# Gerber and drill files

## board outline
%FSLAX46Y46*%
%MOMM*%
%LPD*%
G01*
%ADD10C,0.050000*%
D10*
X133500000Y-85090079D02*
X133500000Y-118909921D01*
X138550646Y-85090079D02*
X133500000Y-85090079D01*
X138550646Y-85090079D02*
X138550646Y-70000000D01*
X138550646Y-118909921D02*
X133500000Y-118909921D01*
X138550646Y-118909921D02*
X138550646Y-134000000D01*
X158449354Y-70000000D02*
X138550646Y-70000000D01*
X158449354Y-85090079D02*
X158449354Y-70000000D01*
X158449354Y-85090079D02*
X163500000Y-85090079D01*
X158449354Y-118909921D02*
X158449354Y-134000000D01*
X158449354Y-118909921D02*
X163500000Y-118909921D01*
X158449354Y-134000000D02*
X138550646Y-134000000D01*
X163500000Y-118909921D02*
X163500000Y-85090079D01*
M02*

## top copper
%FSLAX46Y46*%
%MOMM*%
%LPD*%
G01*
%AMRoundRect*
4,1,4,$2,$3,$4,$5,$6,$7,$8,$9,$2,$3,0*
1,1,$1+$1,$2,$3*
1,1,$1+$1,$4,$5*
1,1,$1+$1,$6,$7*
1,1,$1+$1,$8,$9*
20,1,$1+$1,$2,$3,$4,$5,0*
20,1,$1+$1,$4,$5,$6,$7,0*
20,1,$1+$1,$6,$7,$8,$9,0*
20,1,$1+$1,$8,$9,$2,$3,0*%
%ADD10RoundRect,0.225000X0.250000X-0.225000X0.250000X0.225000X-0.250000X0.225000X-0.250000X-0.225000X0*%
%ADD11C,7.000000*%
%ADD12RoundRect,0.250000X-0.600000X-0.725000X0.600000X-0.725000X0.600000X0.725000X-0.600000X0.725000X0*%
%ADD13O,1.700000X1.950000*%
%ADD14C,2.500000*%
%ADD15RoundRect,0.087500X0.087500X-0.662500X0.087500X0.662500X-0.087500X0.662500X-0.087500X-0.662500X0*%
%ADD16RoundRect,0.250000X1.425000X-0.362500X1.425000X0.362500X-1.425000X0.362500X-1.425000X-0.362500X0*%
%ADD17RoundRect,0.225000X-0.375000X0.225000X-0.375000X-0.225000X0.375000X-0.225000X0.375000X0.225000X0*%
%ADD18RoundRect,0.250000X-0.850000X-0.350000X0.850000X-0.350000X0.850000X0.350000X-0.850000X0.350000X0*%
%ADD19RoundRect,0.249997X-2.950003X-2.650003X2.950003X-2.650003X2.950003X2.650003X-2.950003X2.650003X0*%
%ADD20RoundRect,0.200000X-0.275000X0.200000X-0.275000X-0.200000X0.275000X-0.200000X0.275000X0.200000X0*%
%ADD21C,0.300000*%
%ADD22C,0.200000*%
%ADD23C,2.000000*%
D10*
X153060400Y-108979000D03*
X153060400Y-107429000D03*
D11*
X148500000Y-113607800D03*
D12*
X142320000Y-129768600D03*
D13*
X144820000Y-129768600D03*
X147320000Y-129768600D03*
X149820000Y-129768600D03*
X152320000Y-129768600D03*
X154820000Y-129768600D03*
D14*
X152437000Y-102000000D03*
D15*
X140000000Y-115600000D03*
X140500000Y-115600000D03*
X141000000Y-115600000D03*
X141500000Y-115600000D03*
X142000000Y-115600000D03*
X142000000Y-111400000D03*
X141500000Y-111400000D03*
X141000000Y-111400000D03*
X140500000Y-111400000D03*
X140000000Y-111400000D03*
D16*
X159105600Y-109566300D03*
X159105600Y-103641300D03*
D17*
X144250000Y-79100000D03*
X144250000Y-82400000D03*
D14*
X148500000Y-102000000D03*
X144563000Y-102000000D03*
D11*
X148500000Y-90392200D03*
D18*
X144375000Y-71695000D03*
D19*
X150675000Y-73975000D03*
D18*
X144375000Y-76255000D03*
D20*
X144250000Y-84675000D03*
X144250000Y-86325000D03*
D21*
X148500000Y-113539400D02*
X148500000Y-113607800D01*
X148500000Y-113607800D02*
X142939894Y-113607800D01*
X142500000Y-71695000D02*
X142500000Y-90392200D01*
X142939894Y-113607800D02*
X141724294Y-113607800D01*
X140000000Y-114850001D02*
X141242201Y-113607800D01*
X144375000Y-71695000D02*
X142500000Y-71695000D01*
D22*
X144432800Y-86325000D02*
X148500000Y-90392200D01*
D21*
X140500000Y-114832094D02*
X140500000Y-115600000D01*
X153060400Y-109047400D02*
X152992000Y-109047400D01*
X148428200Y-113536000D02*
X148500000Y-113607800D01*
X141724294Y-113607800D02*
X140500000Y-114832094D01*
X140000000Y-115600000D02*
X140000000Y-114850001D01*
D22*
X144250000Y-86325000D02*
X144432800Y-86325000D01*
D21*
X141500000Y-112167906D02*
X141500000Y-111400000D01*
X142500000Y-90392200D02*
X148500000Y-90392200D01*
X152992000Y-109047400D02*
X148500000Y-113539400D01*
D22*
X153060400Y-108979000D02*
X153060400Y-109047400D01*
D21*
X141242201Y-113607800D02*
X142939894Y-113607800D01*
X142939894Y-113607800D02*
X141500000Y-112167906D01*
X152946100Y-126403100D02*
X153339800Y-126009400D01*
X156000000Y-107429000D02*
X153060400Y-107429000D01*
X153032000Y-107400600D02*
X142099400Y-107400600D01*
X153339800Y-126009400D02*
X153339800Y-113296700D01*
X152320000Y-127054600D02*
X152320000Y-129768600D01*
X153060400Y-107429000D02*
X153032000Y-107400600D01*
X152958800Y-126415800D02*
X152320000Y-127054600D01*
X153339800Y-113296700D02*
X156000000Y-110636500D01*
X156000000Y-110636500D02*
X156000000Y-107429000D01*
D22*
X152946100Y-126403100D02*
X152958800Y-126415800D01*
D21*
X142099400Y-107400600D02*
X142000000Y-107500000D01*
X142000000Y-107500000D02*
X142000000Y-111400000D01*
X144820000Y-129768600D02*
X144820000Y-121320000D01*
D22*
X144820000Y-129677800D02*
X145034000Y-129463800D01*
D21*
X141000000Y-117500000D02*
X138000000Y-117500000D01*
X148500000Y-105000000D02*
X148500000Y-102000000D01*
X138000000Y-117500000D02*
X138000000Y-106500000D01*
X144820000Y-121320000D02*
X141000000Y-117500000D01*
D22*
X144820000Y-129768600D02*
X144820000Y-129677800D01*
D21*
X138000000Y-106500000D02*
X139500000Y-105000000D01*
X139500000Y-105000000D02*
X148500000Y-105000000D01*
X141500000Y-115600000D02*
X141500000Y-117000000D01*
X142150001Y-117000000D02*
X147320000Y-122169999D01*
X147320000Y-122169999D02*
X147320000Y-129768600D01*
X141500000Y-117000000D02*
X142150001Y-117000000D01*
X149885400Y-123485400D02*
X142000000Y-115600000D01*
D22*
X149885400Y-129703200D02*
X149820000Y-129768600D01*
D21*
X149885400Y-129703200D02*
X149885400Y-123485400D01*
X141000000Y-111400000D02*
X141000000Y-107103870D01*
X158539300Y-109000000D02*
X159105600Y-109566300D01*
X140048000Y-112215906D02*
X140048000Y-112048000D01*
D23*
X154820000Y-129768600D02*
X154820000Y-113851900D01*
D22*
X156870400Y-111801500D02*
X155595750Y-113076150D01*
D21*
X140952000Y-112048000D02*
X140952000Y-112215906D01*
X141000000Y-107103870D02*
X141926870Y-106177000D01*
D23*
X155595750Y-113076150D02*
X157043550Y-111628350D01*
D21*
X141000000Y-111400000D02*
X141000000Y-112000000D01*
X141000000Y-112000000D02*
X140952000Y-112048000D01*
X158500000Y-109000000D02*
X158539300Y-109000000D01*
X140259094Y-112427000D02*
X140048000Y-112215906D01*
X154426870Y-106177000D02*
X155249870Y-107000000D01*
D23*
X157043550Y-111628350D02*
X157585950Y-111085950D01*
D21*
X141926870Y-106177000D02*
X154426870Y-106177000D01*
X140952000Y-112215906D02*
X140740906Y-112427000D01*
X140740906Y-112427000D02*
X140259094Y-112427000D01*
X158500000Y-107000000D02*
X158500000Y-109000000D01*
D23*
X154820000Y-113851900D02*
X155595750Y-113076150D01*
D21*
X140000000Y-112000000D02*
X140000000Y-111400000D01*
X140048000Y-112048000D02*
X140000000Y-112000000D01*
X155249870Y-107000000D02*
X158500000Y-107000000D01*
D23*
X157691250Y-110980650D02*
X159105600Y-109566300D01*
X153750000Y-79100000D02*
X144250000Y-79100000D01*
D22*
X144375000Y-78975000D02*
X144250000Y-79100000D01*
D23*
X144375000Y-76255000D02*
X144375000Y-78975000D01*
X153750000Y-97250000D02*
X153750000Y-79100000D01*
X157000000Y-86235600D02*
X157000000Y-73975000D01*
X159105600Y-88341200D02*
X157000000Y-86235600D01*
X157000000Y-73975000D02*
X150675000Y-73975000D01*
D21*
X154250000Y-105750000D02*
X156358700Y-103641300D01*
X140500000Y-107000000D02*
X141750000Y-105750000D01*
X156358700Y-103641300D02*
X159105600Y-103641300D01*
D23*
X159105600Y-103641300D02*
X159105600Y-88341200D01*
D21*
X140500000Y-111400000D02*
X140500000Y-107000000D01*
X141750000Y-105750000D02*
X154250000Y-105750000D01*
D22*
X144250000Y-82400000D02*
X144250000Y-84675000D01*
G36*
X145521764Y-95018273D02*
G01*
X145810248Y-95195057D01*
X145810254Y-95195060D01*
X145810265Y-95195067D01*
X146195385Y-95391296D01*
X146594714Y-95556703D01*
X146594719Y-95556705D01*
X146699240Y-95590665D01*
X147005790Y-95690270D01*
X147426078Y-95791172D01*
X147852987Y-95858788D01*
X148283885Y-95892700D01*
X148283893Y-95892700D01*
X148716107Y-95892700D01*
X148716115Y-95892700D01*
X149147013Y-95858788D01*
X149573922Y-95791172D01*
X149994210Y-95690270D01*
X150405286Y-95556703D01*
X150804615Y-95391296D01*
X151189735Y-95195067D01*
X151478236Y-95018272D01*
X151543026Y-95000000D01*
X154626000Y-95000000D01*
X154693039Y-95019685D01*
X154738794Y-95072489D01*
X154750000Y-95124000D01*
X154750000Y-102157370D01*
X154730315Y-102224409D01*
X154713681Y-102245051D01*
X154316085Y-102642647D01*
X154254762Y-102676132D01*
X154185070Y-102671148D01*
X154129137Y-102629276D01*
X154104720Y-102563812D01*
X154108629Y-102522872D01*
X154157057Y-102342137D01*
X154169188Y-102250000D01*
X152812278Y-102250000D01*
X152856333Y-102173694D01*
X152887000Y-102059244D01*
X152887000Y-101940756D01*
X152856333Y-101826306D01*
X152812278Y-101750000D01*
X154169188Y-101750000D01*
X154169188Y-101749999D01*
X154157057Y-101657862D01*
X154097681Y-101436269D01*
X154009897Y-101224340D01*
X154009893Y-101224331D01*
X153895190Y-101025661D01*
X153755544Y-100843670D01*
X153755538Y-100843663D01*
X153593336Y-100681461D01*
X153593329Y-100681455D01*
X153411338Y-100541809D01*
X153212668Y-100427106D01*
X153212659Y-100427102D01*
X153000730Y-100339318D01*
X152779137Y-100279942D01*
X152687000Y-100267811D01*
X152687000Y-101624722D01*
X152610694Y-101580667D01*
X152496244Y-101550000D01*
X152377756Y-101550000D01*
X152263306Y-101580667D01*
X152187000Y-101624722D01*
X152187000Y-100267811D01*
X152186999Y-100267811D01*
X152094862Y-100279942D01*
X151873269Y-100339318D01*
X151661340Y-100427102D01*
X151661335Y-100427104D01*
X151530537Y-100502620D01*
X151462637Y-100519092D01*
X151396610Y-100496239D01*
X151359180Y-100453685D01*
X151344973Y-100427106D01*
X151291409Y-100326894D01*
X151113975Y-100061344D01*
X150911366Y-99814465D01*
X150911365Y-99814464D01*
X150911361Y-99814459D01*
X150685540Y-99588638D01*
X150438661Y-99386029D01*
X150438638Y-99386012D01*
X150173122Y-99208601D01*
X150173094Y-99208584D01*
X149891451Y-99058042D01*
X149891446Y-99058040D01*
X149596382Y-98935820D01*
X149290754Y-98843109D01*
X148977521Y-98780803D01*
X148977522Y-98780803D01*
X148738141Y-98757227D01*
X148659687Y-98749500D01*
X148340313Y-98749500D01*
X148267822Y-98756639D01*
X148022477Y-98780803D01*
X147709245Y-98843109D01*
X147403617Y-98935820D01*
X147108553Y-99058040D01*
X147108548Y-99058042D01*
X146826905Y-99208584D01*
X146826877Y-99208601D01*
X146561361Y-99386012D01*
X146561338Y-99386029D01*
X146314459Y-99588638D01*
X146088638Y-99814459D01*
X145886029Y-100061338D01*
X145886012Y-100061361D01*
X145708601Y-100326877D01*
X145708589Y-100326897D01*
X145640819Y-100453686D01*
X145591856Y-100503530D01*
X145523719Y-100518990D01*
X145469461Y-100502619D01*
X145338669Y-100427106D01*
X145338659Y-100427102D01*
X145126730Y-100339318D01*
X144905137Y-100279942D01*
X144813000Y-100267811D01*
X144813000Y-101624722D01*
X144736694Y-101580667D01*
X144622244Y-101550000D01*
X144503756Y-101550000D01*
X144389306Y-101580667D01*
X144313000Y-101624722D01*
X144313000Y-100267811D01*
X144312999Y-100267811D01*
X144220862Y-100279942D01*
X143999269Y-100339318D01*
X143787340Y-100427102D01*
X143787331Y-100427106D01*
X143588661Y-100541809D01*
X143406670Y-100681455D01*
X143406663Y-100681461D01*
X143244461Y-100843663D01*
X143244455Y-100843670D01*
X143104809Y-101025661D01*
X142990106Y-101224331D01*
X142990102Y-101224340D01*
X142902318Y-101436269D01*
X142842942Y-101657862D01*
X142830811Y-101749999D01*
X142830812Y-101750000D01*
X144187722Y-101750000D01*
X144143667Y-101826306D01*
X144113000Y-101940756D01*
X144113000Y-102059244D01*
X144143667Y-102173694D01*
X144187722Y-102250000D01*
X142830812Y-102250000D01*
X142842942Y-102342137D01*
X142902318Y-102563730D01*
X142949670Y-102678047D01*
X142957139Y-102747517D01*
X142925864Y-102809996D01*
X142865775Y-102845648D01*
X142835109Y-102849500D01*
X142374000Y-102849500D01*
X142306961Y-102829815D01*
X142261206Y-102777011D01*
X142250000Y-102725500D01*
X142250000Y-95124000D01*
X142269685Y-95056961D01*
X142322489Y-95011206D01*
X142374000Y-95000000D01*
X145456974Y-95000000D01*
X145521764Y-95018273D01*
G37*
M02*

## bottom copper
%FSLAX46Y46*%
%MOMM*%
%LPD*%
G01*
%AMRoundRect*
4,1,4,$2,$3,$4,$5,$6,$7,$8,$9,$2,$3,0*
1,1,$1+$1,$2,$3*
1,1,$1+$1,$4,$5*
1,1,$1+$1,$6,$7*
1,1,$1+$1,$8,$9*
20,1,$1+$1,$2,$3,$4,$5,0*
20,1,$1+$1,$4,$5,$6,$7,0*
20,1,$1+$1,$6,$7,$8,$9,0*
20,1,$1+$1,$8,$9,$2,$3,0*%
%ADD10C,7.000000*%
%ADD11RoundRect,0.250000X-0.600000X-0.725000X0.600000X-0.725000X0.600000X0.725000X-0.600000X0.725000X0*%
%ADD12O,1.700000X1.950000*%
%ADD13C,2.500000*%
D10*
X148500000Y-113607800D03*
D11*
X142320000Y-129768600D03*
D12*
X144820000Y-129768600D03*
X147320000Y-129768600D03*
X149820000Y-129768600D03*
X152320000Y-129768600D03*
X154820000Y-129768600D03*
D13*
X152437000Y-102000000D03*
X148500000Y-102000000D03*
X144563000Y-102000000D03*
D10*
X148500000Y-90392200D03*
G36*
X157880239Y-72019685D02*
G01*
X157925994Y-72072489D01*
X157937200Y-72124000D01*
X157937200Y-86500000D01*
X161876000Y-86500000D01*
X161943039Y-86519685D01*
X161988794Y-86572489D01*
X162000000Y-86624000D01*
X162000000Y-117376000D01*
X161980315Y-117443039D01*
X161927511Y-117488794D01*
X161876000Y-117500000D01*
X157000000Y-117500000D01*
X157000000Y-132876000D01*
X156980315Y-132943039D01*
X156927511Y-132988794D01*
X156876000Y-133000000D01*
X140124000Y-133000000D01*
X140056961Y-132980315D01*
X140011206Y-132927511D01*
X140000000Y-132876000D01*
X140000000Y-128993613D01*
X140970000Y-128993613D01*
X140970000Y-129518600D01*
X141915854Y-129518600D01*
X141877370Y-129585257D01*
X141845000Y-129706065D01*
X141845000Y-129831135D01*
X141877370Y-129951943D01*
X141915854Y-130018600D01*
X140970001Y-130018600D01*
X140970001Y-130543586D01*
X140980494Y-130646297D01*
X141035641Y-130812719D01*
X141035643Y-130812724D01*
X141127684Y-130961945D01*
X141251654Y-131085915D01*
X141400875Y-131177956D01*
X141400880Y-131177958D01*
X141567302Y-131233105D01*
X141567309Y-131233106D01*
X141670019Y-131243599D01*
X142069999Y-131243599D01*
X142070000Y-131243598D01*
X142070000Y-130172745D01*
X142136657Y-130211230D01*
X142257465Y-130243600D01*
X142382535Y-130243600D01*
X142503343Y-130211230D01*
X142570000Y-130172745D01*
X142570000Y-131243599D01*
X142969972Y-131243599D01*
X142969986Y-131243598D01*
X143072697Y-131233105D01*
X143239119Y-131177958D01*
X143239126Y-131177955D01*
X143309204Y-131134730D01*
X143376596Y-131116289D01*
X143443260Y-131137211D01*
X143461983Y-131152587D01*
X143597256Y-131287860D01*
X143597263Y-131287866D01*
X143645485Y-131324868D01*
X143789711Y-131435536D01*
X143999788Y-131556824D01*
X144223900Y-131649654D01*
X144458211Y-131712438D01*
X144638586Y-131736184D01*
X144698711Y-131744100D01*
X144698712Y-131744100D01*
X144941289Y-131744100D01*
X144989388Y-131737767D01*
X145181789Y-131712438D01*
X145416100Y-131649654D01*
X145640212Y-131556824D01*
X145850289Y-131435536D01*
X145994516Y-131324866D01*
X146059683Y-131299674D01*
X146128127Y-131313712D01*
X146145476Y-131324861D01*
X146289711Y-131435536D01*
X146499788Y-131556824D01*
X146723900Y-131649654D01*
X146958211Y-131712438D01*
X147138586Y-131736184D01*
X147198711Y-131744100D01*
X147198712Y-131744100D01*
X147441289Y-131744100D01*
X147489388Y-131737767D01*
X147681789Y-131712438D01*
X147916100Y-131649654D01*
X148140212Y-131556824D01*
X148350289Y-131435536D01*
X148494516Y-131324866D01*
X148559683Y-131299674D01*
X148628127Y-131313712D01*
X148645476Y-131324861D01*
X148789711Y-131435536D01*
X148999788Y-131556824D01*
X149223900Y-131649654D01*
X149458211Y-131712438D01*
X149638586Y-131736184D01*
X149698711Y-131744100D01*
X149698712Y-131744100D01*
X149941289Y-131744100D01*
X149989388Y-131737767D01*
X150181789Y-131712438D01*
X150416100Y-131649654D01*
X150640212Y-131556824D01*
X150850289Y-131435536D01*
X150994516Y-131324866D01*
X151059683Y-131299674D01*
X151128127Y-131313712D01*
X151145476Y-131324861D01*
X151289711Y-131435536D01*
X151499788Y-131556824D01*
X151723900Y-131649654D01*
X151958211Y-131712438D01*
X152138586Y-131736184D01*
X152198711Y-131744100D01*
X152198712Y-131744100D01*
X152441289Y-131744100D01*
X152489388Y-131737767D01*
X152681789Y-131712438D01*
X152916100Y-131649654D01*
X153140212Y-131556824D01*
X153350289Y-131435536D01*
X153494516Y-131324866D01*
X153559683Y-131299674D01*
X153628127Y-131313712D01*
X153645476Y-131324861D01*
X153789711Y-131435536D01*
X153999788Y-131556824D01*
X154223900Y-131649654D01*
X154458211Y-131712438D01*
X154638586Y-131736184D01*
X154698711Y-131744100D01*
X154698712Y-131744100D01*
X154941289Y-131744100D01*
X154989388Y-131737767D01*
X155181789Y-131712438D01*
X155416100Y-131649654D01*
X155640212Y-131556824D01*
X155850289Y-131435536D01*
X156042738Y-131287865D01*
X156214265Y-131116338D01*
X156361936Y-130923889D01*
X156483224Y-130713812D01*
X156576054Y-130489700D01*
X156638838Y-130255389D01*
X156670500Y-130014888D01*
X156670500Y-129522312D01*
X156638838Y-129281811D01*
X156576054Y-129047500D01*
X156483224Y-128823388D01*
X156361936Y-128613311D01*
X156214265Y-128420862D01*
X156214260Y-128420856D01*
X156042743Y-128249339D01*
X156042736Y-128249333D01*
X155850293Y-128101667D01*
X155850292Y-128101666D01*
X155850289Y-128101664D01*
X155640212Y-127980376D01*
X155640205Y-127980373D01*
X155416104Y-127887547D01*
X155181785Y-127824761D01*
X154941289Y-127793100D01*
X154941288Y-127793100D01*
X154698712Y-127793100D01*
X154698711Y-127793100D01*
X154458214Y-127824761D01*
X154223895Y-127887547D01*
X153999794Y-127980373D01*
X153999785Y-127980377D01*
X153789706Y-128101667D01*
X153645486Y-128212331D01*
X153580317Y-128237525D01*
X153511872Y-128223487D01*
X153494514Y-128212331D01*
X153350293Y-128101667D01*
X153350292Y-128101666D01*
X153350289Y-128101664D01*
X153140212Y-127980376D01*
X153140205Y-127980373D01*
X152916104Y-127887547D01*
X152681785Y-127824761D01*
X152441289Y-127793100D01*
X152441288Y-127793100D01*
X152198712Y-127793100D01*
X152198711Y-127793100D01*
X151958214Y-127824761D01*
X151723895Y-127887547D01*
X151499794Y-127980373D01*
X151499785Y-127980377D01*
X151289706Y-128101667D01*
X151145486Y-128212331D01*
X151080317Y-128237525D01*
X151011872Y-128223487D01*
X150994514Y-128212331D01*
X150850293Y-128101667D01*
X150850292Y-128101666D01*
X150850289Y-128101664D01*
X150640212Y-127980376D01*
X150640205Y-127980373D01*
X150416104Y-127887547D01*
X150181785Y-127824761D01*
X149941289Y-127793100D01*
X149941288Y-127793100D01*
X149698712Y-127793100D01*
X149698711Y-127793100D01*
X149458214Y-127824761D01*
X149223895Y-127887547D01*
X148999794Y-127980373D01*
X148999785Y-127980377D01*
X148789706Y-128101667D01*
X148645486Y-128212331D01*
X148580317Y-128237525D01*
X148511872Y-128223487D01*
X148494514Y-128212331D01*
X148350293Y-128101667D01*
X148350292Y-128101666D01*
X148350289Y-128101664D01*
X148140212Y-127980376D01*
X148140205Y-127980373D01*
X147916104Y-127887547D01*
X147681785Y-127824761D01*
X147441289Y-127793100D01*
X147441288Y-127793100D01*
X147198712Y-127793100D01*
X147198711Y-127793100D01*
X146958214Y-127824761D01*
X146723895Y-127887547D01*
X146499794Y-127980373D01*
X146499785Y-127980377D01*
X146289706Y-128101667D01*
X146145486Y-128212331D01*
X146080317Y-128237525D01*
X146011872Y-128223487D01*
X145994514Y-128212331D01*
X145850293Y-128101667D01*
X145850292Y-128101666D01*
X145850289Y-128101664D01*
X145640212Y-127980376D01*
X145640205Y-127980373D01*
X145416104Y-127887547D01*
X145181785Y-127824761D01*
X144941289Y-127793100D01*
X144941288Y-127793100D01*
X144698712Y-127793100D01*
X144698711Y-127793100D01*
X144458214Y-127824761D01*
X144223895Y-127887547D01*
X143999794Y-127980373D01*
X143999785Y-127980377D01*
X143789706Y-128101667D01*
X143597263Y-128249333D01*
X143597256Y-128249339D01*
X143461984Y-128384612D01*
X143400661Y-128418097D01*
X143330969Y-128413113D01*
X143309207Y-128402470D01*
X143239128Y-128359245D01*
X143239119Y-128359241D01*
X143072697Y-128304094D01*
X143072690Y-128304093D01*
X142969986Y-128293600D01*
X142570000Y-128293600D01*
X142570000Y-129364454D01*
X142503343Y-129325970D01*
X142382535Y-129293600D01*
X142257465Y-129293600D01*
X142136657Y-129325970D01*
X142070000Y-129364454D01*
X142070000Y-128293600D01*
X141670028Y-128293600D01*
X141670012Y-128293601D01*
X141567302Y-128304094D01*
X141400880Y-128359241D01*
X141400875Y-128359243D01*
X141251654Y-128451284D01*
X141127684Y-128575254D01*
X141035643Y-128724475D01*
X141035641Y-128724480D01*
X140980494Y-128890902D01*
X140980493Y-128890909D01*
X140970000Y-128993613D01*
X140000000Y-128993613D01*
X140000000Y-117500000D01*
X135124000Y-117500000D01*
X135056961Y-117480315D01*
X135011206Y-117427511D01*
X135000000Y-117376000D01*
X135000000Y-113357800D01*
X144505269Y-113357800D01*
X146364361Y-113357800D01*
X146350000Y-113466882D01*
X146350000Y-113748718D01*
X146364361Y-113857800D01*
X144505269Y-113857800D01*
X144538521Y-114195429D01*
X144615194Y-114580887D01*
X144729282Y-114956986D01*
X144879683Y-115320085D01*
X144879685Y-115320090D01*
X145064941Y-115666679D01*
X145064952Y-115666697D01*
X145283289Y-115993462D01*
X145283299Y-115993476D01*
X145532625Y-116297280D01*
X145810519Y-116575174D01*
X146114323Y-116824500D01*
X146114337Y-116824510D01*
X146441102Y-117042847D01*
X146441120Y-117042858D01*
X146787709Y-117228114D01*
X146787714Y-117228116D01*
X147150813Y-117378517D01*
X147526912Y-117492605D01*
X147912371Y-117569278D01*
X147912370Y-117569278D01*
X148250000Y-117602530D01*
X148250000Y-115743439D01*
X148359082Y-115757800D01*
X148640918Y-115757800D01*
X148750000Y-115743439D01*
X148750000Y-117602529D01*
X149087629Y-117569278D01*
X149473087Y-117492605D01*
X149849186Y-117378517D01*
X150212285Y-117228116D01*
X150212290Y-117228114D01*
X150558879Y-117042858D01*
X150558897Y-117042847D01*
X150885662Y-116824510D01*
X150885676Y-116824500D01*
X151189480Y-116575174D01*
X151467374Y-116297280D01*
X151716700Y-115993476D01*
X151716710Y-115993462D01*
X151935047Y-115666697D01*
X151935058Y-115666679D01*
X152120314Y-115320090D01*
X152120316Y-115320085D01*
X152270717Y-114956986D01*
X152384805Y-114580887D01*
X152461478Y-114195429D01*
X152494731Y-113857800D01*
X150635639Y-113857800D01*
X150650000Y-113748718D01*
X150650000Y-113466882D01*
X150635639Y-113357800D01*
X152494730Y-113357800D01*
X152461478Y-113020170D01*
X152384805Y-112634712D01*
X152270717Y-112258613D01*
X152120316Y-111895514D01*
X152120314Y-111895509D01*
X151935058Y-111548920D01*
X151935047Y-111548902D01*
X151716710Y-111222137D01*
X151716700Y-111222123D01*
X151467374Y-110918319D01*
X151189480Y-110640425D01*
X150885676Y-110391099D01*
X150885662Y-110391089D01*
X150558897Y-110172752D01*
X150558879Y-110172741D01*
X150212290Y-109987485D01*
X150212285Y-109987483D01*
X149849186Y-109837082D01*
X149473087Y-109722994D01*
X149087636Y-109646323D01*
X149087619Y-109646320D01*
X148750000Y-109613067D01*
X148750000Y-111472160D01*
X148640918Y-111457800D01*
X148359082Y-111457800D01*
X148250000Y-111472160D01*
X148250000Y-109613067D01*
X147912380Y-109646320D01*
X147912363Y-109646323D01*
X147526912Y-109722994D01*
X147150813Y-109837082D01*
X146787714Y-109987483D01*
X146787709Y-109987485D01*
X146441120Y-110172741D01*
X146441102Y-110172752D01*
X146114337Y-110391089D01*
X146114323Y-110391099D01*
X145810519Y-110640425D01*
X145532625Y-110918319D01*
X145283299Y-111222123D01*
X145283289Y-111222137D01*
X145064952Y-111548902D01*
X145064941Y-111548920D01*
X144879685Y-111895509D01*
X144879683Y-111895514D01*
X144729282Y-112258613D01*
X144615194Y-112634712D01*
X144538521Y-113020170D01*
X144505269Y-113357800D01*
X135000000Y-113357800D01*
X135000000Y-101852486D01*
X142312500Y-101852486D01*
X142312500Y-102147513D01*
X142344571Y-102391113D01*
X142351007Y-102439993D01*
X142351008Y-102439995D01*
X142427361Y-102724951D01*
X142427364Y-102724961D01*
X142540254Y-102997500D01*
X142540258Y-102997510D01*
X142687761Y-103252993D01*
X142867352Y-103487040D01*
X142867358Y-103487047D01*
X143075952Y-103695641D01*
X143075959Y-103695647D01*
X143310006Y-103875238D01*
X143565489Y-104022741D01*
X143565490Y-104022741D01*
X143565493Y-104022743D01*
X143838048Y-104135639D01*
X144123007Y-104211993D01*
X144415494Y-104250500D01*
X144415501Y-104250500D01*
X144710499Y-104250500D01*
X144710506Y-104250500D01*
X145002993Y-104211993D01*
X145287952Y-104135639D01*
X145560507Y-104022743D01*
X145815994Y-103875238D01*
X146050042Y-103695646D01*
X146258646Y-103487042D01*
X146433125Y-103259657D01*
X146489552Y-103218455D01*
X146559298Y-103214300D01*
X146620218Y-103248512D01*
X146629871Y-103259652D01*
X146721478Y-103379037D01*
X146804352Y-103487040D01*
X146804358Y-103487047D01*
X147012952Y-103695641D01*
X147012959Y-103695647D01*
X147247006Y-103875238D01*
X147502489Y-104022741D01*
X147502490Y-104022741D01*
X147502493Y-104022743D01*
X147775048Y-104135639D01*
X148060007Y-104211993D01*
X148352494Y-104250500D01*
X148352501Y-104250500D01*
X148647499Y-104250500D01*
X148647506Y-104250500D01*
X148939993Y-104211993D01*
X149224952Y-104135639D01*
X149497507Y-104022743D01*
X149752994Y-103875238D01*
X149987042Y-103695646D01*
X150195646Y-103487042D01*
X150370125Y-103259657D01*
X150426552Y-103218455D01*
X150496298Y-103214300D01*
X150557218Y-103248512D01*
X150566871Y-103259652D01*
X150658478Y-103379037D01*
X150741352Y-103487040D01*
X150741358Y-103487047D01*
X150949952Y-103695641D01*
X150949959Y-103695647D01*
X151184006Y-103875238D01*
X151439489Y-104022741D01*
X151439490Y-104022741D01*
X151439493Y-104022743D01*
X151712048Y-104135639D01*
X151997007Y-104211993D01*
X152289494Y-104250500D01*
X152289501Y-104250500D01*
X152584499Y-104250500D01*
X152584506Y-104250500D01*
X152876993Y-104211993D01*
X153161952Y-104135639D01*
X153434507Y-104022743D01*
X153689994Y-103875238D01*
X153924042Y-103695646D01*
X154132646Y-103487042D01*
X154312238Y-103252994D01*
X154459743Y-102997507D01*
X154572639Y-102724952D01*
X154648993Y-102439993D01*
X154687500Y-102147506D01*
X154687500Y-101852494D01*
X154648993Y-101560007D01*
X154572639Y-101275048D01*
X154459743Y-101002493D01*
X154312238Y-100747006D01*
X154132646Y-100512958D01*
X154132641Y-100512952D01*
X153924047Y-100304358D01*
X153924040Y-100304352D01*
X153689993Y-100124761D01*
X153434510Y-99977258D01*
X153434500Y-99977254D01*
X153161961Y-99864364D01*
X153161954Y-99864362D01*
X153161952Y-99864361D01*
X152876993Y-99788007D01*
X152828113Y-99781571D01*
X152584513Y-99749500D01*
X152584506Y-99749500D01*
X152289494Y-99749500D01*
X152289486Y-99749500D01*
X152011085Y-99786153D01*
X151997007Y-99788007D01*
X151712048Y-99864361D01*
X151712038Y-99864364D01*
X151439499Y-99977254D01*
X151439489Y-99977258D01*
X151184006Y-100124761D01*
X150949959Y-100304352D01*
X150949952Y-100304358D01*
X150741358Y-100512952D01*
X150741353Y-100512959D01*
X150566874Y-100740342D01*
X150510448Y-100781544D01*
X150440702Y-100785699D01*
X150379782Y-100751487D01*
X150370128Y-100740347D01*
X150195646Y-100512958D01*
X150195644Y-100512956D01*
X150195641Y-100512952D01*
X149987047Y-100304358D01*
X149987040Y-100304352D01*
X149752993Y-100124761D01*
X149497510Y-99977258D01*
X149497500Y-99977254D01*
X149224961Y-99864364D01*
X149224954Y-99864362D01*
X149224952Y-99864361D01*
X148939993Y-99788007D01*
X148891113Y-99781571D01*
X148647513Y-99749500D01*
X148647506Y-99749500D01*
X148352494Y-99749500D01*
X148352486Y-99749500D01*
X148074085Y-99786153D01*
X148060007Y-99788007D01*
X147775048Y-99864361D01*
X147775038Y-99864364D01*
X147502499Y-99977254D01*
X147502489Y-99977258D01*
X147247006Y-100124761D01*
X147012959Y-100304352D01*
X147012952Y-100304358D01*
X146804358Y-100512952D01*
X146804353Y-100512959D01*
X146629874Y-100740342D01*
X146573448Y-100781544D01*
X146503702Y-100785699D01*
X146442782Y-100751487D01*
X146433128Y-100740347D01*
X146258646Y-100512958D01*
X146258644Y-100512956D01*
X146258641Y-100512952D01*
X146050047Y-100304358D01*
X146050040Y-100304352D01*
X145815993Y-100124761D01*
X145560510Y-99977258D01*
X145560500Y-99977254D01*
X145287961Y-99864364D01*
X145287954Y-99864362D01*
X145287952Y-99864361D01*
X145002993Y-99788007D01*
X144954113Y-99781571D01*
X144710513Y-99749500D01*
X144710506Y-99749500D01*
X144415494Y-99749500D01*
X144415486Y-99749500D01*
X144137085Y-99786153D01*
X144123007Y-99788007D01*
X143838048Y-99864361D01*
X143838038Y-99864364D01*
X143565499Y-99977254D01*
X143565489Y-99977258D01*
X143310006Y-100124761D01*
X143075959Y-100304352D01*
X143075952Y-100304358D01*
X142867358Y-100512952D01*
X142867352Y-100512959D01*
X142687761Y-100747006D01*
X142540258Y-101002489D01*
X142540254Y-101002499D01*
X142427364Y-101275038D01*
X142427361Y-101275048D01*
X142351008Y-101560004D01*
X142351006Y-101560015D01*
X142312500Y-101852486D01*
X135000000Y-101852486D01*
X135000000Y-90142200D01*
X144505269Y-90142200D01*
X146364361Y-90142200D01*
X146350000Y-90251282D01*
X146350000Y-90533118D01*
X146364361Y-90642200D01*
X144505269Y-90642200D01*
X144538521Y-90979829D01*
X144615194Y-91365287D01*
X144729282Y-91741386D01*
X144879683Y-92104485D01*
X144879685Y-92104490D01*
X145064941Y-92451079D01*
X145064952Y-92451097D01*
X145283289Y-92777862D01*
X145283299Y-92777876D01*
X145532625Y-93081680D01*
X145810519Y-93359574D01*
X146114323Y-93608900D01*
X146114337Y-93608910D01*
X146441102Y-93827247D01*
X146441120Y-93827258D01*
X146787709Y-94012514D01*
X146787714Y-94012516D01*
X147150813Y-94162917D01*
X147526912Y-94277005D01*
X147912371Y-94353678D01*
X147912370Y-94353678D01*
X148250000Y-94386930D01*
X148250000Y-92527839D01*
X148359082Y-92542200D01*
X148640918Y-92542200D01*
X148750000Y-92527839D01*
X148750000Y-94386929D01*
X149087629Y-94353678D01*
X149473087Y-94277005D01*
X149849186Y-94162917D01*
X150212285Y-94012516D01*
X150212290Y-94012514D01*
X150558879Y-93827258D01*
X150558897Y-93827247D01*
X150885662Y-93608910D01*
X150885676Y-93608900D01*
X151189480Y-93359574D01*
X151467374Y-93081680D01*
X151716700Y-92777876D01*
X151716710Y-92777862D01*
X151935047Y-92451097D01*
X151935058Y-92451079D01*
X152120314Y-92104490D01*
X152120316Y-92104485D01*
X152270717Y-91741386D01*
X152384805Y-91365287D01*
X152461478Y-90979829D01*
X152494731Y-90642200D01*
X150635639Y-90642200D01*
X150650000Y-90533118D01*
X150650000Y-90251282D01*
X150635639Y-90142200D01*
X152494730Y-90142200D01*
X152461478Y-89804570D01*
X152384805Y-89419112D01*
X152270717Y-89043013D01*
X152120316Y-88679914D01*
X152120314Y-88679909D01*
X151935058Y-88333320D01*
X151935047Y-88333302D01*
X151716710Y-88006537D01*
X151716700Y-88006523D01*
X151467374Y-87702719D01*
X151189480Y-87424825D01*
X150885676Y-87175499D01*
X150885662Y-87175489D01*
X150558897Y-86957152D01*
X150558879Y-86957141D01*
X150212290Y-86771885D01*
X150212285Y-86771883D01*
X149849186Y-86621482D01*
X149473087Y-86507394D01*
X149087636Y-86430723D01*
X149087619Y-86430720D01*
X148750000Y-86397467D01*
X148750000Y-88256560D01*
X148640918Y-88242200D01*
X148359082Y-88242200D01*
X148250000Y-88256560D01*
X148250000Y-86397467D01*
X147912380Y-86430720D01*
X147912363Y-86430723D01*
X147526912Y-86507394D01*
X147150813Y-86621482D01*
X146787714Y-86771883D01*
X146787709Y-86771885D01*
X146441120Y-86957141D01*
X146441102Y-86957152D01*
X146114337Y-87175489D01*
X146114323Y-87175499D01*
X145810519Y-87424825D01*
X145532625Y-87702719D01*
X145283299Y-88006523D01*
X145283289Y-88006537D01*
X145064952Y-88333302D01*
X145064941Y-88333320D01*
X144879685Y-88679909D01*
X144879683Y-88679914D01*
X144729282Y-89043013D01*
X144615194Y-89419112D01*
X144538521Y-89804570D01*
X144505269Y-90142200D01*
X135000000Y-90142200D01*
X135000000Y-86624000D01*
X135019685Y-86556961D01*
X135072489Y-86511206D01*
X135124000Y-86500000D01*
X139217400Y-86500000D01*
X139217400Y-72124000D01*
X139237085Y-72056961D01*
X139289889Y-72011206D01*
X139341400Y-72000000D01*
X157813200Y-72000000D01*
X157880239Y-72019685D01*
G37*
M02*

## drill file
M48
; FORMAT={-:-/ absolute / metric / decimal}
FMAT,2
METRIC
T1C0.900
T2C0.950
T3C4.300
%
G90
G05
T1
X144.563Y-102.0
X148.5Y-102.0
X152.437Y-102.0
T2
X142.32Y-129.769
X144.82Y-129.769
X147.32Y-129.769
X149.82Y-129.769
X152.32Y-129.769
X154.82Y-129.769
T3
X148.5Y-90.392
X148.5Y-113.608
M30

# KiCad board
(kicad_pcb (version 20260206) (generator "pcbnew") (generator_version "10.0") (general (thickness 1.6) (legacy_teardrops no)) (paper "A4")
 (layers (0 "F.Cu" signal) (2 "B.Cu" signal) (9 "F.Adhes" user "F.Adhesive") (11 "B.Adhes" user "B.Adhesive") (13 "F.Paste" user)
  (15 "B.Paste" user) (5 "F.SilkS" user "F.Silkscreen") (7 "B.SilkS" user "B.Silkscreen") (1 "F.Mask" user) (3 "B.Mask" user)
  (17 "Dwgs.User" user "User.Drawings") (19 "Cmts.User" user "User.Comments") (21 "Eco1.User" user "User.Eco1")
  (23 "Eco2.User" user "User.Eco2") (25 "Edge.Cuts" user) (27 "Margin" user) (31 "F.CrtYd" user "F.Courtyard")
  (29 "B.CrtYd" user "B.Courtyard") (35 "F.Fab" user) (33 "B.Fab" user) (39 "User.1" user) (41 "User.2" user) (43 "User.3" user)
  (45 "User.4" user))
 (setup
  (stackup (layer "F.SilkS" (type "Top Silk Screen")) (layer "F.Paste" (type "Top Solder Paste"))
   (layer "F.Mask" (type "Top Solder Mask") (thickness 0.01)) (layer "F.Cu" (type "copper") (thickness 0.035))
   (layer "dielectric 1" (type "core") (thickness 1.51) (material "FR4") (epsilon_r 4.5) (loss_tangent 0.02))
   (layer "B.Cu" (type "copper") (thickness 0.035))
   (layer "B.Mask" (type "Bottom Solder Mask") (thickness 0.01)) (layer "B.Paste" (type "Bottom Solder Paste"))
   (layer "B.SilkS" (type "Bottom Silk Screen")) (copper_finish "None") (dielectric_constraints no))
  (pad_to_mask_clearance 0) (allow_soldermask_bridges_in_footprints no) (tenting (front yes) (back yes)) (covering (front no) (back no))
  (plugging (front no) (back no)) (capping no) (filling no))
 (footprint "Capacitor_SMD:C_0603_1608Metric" (layer "F.Cu") (at 153.0604 108.204 90)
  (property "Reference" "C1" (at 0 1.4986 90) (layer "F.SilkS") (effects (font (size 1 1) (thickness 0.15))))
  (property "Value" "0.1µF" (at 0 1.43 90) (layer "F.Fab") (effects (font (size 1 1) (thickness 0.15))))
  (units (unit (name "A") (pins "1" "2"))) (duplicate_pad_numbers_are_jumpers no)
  (pad "1" smd roundrect (at -0.775 0 90) (size 0.9 0.95) (layers "F.Cu" "F.Mask" "F.Paste") (roundrect_rratio 0.25) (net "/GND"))
  (pad "2" smd roundrect (at 0.775 0 90) (size 0.9 0.95) (layers "F.Cu" "F.Mask" "F.Paste") (roundrect_rratio 0.25) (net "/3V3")))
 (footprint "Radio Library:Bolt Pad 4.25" (layer "F.Cu") (at 148.5 113.6078)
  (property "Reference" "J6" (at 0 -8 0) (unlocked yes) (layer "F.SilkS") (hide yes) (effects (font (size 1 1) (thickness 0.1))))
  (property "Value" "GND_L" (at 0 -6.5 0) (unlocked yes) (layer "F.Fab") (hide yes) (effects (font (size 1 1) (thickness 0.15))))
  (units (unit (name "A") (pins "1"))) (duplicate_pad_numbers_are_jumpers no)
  (pad "1" thru_hole circle (at 0 0) (size 7 7) (drill 4.3) (layers "*.Cu" "*.Mask") (remove_unused_layers no) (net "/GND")
   (thermal_bridge_angle 90)))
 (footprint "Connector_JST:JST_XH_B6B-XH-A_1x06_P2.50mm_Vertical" (layer "F.Cu") (at 142.32 129.7686)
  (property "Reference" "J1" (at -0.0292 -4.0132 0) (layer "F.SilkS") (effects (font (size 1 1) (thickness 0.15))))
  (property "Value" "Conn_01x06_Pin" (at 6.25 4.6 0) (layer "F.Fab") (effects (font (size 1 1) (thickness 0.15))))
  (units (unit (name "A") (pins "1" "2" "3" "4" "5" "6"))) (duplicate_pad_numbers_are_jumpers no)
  (pad "1" thru_hole roundrect (at 0 0) (size 1.7 1.95) (drill 0.95) (layers "*.Cu" "*.Mask") (remove_unused_layers no)
   (roundrect_rratio 0.147059) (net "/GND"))
  (pad "2" thru_hole oval (at 2.5 0) (size 1.7 1.95) (drill 0.95) (layers "*.Cu" "*.Mask") (remove_unused_layers no) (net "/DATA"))
  (pad "3" thru_hole oval (at 5 0) (size 1.7 1.95) (drill 0.95) (layers "*.Cu" "*.Mask") (remove_unused_layers no) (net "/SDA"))
  (pad "4" thru_hole oval (at 7.5 0) (size 1.7 1.95) (drill 0.95) (layers "*.Cu" "*.Mask") (remove_unused_layers no) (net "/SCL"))
  (pad "5" thru_hole oval (at 10 0) (size 1.7 1.95) (drill 0.95) (layers "*.Cu" "*.Mask") (remove_unused_layers no) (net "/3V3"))
  (pad "6" thru_hole oval (at 12.5 0) (size 1.7 1.95) (drill 0.95) (layers "*.Cu" "*.Mask") (remove_unused_layers no) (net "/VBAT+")))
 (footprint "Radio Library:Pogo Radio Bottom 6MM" (layer "F.Cu") (at 152.437 102)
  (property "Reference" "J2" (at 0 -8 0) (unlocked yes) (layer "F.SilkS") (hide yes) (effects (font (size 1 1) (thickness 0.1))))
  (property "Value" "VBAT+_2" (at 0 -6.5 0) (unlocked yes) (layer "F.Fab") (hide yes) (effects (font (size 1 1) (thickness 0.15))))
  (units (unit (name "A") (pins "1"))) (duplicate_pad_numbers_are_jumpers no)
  (pad "1" thru_hole circle (at 0 0) (size 2.5 2.5) (drill 0.9) (layers "*.Cu" "*.Mask") (remove_unused_layers no) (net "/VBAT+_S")
   (thermal_bridge_angle 90)))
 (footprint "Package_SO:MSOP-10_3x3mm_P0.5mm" (layer "F.Cu") (at 141 113.5 90)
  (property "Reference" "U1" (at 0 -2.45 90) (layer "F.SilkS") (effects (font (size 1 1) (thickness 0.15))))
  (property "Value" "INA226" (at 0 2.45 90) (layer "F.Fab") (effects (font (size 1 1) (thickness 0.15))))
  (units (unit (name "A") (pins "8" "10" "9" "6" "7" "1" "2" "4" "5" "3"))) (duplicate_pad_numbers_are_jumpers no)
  (pad "1" smd roundrect (at -2.1 -1 90) (size 1.5 0.35) (layers "F.Cu" "F.Mask" "F.Paste") (roundrect_rratio 0.25) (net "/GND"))
  (pad "2" smd roundrect (at -2.1 -0.5 90) (size 1.5 0.35) (layers "F.Cu" "F.Mask" "F.Paste") (roundrect_rratio 0.25) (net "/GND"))
  (pad "3" smd roundrect (at -2.1 0 90) (size 1.5 0.35) (layers "F.Cu" "F.Mask" "F.Paste") (roundrect_rratio 0.25)
   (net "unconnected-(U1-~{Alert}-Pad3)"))
  (pad "4" smd roundrect (at -2.1 0.5 90) (size 1.5 0.35) (layers "F.Cu" "F.Mask" "F.Paste") (roundrect_rratio 0.25) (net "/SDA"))
  (pad "5" smd roundrect (at -2.1 1 90) (size 1.5 0.35) (layers "F.Cu" "F.Mask" "F.Paste") (roundrect_rratio 0.25) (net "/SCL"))
  (pad "6" smd roundrect (at 2.1 1 90) (size 1.5 0.35) (layers "F.Cu" "F.Mask" "F.Paste") (roundrect_rratio 0.25) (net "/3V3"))
  (pad "7" smd roundrect (at 2.1 0.5 90) (size 1.5 0.35) (layers "F.Cu" "F.Mask" "F.Paste") (roundrect_rratio 0.25) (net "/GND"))
  (pad "8" smd roundrect (at 2.1 0 90) (size 1.5 0.35) (layers "F.Cu" "F.Mask" "F.Paste") (roundrect_rratio 0.25) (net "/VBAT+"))
  (pad "9" smd roundrect (at 2.1 -0.5 90) (size 1.5 0.35) (layers "F.Cu" "F.Mask" "F.Paste") (roundrect_rratio 0.25) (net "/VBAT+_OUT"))
  (pad "10" smd roundrect (at 2.1 -1 90) (size 1.5 0.35) (layers "F.Cu" "F.Mask" "F.Paste") (roundrect_rratio 0.25) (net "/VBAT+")))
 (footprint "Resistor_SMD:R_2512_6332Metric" (layer "F.Cu") (at 159.1056 106.6038 90)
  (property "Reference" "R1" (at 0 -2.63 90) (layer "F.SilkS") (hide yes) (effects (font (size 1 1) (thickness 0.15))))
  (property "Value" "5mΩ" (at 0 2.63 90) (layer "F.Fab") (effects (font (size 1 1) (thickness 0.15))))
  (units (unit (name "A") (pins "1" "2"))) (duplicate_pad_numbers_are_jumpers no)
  (pad "1" smd roundrect (at -2.9625 0 90) (size 1.225 3.35) (layers "F.Cu" "F.Mask" "F.Paste") (roundrect_rratio 0.204082) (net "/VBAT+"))
  (pad "2" smd roundrect (at 2.9625 0 90) (size 1.225 3.35) (layers "F.Cu" "F.Mask" "F.Paste") (roundrect_rratio 0.204082)
   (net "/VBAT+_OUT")))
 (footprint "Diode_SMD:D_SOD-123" (layer "F.Cu") (at 144.25 80.75 -90)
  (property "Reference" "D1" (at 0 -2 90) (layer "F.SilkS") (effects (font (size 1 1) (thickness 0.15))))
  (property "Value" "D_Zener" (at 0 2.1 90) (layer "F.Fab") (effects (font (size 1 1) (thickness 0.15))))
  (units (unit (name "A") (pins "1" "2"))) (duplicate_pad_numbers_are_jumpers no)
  (pad "1" smd roundrect (at -1.65 0 270) (size 0.9 1.2) (layers "F.Cu" "F.Mask" "F.Paste") (roundrect_rratio 0.25) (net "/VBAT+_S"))
  (pad "2" smd roundrect (at 1.65 0 270) (size 0.9 1.2) (layers "F.Cu" "F.Mask" "F.Paste") (roundrect_rratio 0.25) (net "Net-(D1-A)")))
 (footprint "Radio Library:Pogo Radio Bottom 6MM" (layer "F.Cu") (at 148.5 102)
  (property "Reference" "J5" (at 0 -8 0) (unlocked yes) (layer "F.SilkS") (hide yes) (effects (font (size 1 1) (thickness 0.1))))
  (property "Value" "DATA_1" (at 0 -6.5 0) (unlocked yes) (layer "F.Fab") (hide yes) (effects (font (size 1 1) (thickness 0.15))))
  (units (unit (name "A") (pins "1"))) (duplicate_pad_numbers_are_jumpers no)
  (pad "1" thru_hole circle (at 0 0) (size 2.5 2.5) (drill 0.9) (layers "*.Cu" "*.Mask") (remove_unused_layers no) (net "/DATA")
   (thermal_bridge_angle 90)))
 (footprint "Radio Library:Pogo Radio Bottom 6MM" (layer "F.Cu") (at 144.563 102)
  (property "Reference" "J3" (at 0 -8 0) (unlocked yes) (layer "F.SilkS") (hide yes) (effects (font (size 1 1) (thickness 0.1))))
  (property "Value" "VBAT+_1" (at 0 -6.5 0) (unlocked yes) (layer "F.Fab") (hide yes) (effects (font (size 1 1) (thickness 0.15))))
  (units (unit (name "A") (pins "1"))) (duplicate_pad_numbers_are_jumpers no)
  (pad "1" thru_hole circle (at 0 0) (size 2.5 2.5) (drill 0.9) (layers "*.Cu" "*.Mask") (remove_unused_layers no) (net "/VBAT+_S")
   (thermal_bridge_angle 90)))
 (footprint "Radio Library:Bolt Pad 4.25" (layer "F.Cu") (at 148.5 90.3922)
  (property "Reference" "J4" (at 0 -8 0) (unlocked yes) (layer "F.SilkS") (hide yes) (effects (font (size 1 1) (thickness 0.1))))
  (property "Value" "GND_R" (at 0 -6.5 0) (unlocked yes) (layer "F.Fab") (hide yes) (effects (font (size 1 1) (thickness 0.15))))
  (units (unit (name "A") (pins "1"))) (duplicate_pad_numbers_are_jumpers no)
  (pad "1" thru_hole circle (at 0 0) (size 7 7) (drill 4.3) (layers "*.Cu" "*.Mask") (remove_unused_layers no) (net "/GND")
   (thermal_bridge_angle 90)))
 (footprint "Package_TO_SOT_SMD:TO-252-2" (layer "F.Cu") (at 149.415 73.975)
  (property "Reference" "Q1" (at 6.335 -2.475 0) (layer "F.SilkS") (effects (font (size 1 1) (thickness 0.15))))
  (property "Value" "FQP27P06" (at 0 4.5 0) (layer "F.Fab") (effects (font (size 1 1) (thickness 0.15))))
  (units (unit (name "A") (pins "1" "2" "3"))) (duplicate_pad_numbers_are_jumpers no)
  (pad "" smd roundrect (at -0.415 -1.525) (size 3.05 2.75) (layers "F.Paste") (roundrect_rratio 0.090909))
  (pad "" smd roundrect (at -0.415 1.525) (size 3.05 2.75) (layers "F.Paste") (roundrect_rratio 0.090909))
  (pad "" smd roundrect (at 2.935 -1.525) (size 3.05 2.75) (layers "F.Paste") (roundrect_rratio 0.090909))
  (pad "" smd roundrect (at 2.935 1.525) (size 3.05 2.75) (layers "F.Paste") (roundrect_rratio 0.090909))
  (pad "1" smd roundrect (at -5.04 -2.28) (size 2.2 1.2) (layers "F.Cu" "F.Mask" "F.Paste") (roundrect_rratio 0.208333) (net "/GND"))
  (pad "2" smd roundrect (at 1.26 0) (size 6.4 5.8) (layers "F.Cu" "F.Mask") (roundrect_rratio 0.043103) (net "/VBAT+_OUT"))
  (pad "3" smd roundrect (at -5.04 2.28) (size 2.2 1.2) (layers "F.Cu" "F.Mask" "F.Paste") (roundrect_rratio 0.208333) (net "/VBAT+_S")))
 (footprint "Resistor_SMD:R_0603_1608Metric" (layer "F.Cu") (at 144.25 85.5 -90)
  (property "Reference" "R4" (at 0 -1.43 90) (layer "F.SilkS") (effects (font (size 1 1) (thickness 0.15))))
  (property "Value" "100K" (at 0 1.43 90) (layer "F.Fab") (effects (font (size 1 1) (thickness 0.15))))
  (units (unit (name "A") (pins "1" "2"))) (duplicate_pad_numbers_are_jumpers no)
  (pad "1" smd roundrect (at -0.825 0 270) (size 0.8 0.95) (layers "F.Cu" "F.Mask" "F.Paste") (roundrect_rratio 0.25) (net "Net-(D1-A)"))
  (pad "2" smd roundrect (at 0.825 0 270) (size 0.8 0.95) (layers "F.Cu" "F.Mask" "F.Paste") (roundrect_rratio 0.25) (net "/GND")))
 (gr_line (start 133.5 85.090079) (end 133.5 118.909921) (stroke (width 0.05) (type default)) (layer "Edge.Cuts"))
 (gr_line (start 138.550646 85.090079) (end 133.5 85.090079) (stroke (width 0.05) (type default)) (layer "Edge.Cuts"))
 (gr_line (start 138.550646 85.090079) (end 138.550646 70) (stroke (width 0.05) (type default)) (layer "Edge.Cuts"))
 (gr_line (start 138.550646 118.909921) (end 133.5 118.909921) (stroke (width 0.05) (type default)) (layer "Edge.Cuts"))
 (gr_line (start 138.550646 118.909921) (end 138.550646 134) (stroke (width 0.05) (type default)) (layer "Edge.Cuts"))
 (gr_line (start 158.449354 70) (end 138.550646 70) (stroke (width 0.05) (type default)) (layer "Edge.Cuts"))
 (gr_line (start 158.449354 85.090079) (end 158.449354 70) (stroke (width 0.05) (type default)) (layer "Edge.Cuts"))
 (gr_line (start 158.449354 85.090079) (end 163.5 85.090079) (stroke (width 0.05) (type default)) (layer "Edge.Cuts"))
 (gr_line (start 158.449354 118.909921) (end 158.449354 134) (stroke (width 0.05) (type default)) (layer "Edge.Cuts"))
 (gr_line (start 158.449354 118.909921) (end 163.5 118.909921) (stroke (width 0.05) (type default)) (layer "Edge.Cuts"))
 (gr_line (start 158.449354 134) (end 138.550646 134) (stroke (width 0.05) (type default)) (layer "Edge.Cuts"))
 (gr_line (start 163.5 118.909921) (end 163.5 85.090079) (stroke (width 0.05) (type default)) (layer "Edge.Cuts"))
 (segment (start 148.5 113.5394) (end 148.5 113.6078) (width 0.3) (layer "F.Cu") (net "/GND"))
 (segment (start 148.5 113.6078) (end 142.939894 113.6078) (width 0.3) (layer "F.Cu") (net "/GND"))
 (segment (start 142.5 71.695) (end 142.5 90.3922) (width 0.3) (layer "F.Cu") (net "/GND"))
 (segment (start 142.939894 113.6078) (end 141.724294 113.6078) (width 0.3) (layer "F.Cu") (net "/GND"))
 (segment (start 140 114.850001) (end 141.242201 113.6078) (width 0.3) (layer "F.Cu") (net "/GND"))
 (segment (start 144.375 71.695) (end 142.5 71.695) (width 0.3) (layer "F.Cu") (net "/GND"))
 (segment (start 144.4328 86.325) (end 148.5 90.3922) (width 0.2) (layer "F.Cu") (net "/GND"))
 (segment (start 140.5 114.832094) (end 140.5 115.6) (width 0.3) (layer "F.Cu") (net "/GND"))
 (segment (start 153.0604 109.0474) (end 152.992 109.0474) (width 0.3) (layer "F.Cu") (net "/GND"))
 (segment (start 148.4282 113.536) (end 148.5 113.6078) (width 0.3) (layer "F.Cu") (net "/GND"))
 (segment (start 141.724294 113.6078) (end 140.5 114.832094) (width 0.3) (layer "F.Cu") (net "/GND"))
 (segment (start 140 115.6) (end 140 114.850001) (width 0.3) (layer "F.Cu") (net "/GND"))
 (segment (start 144.25 86.325) (end 144.4328 86.325) (width 0.2) (layer "F.Cu") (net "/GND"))
 (segment (start 141.5 112.167906) (end 141.5 111.4) (width 0.3) (layer "F.Cu") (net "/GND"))
 (segment (start 142.5 90.3922) (end 148.5 90.3922) (width 0.3) (layer "F.Cu") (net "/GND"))
 (segment (start 152.992 109.0474) (end 148.5 113.5394) (width 0.3) (layer "F.Cu") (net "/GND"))
 (segment (start 153.0604 108.979) (end 153.0604 109.0474) (width 0.2) (layer "F.Cu") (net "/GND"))
 (segment (start 141.242201 113.6078) (end 142.939894 113.6078) (width 0.3) (layer "F.Cu") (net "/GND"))
 (segment (start 142.939894 113.6078) (end 141.5 112.167906) (width 0.3) (layer "F.Cu") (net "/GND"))
 (segment (start 152.9461 126.4031) (end 153.3398 126.0094) (width 0.3) (layer "F.Cu") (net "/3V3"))
 (segment (start 156 107.429) (end 153.0604 107.429) (width 0.3) (layer "F.Cu") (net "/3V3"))
 (segment (start 153.032 107.4006) (end 142.0994 107.4006) (width 0.3) (layer "F.Cu") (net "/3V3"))
 (segment (start 153.3398 126.0094) (end 153.3398 113.2967) (width 0.3) (layer "F.Cu") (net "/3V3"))
 (segment (start 152.32 127.0546) (end 152.32 129.7686) (width 0.3) (layer "F.Cu") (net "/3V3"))
 (segment (start 153.0604 107.429) (end 153.032 107.4006) (width 0.3) (layer "F.Cu") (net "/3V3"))
 (segment (start 152.9588 126.4158) (end 152.32 127.0546) (width 0.3) (layer "F.Cu") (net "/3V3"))
 (segment (start 153.3398 113.2967) (end 156 110.6365) (width 0.3) (layer "F.Cu") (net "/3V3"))
 (segment (start 156 110.6365) (end 156 107.429) (width 0.3) (layer "F.Cu") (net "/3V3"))
 (segment (start 152.9461 126.4031) (end 152.9588 126.4158) (width 0.2) (layer "F.Cu") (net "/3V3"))
 (segment (start 142.0994 107.4006) (end 142 107.5) (width 0.3) (layer "F.Cu") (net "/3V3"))
 (segment (start 142 107.5) (end 142 111.4) (width 0.3) (layer "F.Cu") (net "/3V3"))
 (segment (start 144.82 129.7686) (end 144.82 121.32) (width 0.3) (layer "F.Cu") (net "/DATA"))
 (segment (start 144.82 129.6778) (end 145.034 129.4638) (width 0.2) (layer "F.Cu") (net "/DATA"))
 (segment (start 141 117.5) (end 138 117.5) (width 0.3) (layer "F.Cu") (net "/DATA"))
 (segment (start 148.5 105) (end 148.5 102) (width 0.3) (layer "F.Cu") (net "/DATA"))
 (segment (start 138 117.5) (end 138 106.5) (width 0.3) (layer "F.Cu") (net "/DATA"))
 (segment (start 144.82 121.32) (end 141 117.5) (width 0.3) (layer "F.Cu") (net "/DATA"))
 (segment (start 144.82 129.7686) (end 144.82 129.6778) (width 0.2) (layer "F.Cu") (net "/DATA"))
 (segment (start 138 106.5) (end 139.5 105) (width 0.3) (layer "F.Cu") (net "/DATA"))
 (segment (start 139.5 105) (end 148.5 105) (width 0.3) (layer "F.Cu") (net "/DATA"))
 (segment (start 141.5 115.6) (end 141.5 117) (width 0.3) (layer "F.Cu") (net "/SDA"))
 (segment (start 142.150001 117) (end 147.32 122.169999) (width 0.3) (layer "F.Cu") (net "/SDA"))
 (segment (start 147.32 122.169999) (end 147.32 129.7686) (width 0.3) (layer "F.Cu") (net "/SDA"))
 (segment (start 141.5 117) (end 142.150001 117) (width 0.3) (layer "F.Cu") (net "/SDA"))
 (segment (start 149.8854 123.4854) (end 142 115.6) (width 0.3) (layer "F.Cu") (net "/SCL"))
 (segment (start 149.8854 129.7032) (end 149.82 129.7686) (width 0.2) (layer "F.Cu") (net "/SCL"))
 (segment (start 149.8854 129.7032) (end 149.8854 123.4854) (width 0.3) (layer "F.Cu") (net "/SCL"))
 (segment (start 141 111.4) (end 141 107.10387) (width 0.3) (layer "F.Cu") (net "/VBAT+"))
 (segment (start 158.5393 109) (end 159.1056 109.5663) (width 0.3) (layer "F.Cu") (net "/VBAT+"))
 (segment (start 140.048 112.215906) (end 140.048 112.048) (width 0.3) (layer "F.Cu") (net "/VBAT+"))
 (segment (start 154.82 129.7686) (end 154.82 113.8519) (width 2) (layer "F.Cu") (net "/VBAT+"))
 (segment (start 156.8704 111.8015) (end 155.59575 113.07615) (width 0.2) (layer "F.Cu") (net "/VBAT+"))
 (segment (start 140.952 112.048) (end 140.952 112.215906) (width 0.3) (layer "F.Cu") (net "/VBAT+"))
 (segment (start 141 107.10387) (end 141.92687 106.177) (width 0.3) (layer "F.Cu") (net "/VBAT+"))
 (segment (start 155.59575 113.07615) (end 157.04355 111.62835) (width 2) (layer "F.Cu") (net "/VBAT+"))
 (segment (start 141 111.4) (end 141 112) (width 0.3) (layer "F.Cu") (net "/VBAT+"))
 (segment (start 141 112) (end 140.952 112.048) (width 0.3) (layer "F.Cu") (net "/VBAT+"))
 (segment (start 158.5 109) (end 158.5393 109) (width 0.3) (layer "F.Cu") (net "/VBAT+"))
 (segment (start 140.259094 112.427) (end 140.048 112.215906) (width 0.3) (layer "F.Cu") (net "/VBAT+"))
 (segment (start 154.42687 106.177) (end 155.24987 107) (width 0.3) (layer "F.Cu") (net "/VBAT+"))
 (segment (start 157.04355 111.62835) (end 157.58595 111.08595) (width 2) (layer "F.Cu") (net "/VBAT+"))
 (segment (start 141.92687 106.177) (end 154.42687 106.177) (width 0.3) (layer "F.Cu") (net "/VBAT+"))
 (segment (start 140.952 112.215906) (end 140.740906 112.427) (width 0.3) (layer "F.Cu") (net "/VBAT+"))
 (segment (start 140.740906 112.427) (end 140.259094 112.427) (width 0.3) (layer "F.Cu") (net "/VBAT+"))
 (segment (start 158.5 107) (end 158.5 109) (width 0.3) (layer "F.Cu") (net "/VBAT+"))
 (segment (start 154.82 113.8519) (end 155.59575 113.07615) (width 2) (layer "F.Cu") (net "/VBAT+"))
 (segment (start 140 112) (end 140 111.4) (width 0.3) (layer "F.Cu") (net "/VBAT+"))
 (segment (start 140.048 112.048) (end 140 112) (width 0.3) (layer "F.Cu") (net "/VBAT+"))
 (segment (start 155.24987 107) (end 158.5 107) (width 0.3) (layer "F.Cu") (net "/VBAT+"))
 (segment (start 157.69125 110.98065) (end 159.1056 109.5663) (width 2) (layer "F.Cu") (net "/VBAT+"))
 (segment (start 153.75 79.1) (end 144.25 79.1) (width 2) (layer "F.Cu") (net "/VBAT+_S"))
 (segment (start 144.375 78.975) (end 144.25 79.1) (width 0.2) (layer "F.Cu") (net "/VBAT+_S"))
 (segment (start 144.375 76.255) (end 144.375 78.975) (width 2) (layer "F.Cu") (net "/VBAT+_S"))
 (segment (start 153.75 97.25) (end 153.75 79.1) (width 2) (layer "F.Cu") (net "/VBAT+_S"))
 (segment (start 157 86.2356) (end 157 73.975) (width 2) (layer "F.Cu") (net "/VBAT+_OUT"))
 (segment (start 159.1056 88.3412) (end 157 86.2356) (width 2) (layer "F.Cu") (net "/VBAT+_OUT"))
 (segment (start 157 73.975) (end 150.675 73.975) (width 2) (layer "F.Cu") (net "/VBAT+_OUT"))
 (segment (start 154.25 105.75) (end 156.3587 103.6413) (width 0.3) (layer "F.Cu") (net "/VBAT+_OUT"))
 (segment (start 140.5 107) (end 141.75 105.75) (width 0.3) (layer "F.Cu") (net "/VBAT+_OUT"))
 (segment (start 156.3587 103.6413) (end 159.1056 103.6413) (width 0.3) (layer "F.Cu") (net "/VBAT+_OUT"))
 (segment (start 159.1056 103.6413) (end 159.1056 88.3412) (width 2) (layer "F.Cu") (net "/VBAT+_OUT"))
 (segment (start 140.5 111.4) (end 140.5 107) (width 0.3) (layer "F.Cu") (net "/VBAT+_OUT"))
 (segment (start 141.75 105.75) (end 154.25 105.75) (width 0.3) (layer "F.Cu") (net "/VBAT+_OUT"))
 (segment (start 144.25 82.4) (end 144.25 84.675) (width 0.2) (layer "F.Cu") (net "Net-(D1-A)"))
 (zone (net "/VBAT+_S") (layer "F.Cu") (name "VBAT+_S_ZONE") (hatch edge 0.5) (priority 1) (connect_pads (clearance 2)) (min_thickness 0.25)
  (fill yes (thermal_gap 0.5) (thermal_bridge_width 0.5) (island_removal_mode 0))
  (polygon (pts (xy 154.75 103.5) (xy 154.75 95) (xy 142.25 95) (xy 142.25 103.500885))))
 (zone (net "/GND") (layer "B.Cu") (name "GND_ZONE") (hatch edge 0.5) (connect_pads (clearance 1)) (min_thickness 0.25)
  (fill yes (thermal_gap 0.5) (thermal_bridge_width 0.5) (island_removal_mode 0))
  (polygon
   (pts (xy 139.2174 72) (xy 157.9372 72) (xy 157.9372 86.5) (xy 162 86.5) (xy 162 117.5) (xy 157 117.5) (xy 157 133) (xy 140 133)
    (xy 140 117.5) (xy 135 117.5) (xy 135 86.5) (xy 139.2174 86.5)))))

